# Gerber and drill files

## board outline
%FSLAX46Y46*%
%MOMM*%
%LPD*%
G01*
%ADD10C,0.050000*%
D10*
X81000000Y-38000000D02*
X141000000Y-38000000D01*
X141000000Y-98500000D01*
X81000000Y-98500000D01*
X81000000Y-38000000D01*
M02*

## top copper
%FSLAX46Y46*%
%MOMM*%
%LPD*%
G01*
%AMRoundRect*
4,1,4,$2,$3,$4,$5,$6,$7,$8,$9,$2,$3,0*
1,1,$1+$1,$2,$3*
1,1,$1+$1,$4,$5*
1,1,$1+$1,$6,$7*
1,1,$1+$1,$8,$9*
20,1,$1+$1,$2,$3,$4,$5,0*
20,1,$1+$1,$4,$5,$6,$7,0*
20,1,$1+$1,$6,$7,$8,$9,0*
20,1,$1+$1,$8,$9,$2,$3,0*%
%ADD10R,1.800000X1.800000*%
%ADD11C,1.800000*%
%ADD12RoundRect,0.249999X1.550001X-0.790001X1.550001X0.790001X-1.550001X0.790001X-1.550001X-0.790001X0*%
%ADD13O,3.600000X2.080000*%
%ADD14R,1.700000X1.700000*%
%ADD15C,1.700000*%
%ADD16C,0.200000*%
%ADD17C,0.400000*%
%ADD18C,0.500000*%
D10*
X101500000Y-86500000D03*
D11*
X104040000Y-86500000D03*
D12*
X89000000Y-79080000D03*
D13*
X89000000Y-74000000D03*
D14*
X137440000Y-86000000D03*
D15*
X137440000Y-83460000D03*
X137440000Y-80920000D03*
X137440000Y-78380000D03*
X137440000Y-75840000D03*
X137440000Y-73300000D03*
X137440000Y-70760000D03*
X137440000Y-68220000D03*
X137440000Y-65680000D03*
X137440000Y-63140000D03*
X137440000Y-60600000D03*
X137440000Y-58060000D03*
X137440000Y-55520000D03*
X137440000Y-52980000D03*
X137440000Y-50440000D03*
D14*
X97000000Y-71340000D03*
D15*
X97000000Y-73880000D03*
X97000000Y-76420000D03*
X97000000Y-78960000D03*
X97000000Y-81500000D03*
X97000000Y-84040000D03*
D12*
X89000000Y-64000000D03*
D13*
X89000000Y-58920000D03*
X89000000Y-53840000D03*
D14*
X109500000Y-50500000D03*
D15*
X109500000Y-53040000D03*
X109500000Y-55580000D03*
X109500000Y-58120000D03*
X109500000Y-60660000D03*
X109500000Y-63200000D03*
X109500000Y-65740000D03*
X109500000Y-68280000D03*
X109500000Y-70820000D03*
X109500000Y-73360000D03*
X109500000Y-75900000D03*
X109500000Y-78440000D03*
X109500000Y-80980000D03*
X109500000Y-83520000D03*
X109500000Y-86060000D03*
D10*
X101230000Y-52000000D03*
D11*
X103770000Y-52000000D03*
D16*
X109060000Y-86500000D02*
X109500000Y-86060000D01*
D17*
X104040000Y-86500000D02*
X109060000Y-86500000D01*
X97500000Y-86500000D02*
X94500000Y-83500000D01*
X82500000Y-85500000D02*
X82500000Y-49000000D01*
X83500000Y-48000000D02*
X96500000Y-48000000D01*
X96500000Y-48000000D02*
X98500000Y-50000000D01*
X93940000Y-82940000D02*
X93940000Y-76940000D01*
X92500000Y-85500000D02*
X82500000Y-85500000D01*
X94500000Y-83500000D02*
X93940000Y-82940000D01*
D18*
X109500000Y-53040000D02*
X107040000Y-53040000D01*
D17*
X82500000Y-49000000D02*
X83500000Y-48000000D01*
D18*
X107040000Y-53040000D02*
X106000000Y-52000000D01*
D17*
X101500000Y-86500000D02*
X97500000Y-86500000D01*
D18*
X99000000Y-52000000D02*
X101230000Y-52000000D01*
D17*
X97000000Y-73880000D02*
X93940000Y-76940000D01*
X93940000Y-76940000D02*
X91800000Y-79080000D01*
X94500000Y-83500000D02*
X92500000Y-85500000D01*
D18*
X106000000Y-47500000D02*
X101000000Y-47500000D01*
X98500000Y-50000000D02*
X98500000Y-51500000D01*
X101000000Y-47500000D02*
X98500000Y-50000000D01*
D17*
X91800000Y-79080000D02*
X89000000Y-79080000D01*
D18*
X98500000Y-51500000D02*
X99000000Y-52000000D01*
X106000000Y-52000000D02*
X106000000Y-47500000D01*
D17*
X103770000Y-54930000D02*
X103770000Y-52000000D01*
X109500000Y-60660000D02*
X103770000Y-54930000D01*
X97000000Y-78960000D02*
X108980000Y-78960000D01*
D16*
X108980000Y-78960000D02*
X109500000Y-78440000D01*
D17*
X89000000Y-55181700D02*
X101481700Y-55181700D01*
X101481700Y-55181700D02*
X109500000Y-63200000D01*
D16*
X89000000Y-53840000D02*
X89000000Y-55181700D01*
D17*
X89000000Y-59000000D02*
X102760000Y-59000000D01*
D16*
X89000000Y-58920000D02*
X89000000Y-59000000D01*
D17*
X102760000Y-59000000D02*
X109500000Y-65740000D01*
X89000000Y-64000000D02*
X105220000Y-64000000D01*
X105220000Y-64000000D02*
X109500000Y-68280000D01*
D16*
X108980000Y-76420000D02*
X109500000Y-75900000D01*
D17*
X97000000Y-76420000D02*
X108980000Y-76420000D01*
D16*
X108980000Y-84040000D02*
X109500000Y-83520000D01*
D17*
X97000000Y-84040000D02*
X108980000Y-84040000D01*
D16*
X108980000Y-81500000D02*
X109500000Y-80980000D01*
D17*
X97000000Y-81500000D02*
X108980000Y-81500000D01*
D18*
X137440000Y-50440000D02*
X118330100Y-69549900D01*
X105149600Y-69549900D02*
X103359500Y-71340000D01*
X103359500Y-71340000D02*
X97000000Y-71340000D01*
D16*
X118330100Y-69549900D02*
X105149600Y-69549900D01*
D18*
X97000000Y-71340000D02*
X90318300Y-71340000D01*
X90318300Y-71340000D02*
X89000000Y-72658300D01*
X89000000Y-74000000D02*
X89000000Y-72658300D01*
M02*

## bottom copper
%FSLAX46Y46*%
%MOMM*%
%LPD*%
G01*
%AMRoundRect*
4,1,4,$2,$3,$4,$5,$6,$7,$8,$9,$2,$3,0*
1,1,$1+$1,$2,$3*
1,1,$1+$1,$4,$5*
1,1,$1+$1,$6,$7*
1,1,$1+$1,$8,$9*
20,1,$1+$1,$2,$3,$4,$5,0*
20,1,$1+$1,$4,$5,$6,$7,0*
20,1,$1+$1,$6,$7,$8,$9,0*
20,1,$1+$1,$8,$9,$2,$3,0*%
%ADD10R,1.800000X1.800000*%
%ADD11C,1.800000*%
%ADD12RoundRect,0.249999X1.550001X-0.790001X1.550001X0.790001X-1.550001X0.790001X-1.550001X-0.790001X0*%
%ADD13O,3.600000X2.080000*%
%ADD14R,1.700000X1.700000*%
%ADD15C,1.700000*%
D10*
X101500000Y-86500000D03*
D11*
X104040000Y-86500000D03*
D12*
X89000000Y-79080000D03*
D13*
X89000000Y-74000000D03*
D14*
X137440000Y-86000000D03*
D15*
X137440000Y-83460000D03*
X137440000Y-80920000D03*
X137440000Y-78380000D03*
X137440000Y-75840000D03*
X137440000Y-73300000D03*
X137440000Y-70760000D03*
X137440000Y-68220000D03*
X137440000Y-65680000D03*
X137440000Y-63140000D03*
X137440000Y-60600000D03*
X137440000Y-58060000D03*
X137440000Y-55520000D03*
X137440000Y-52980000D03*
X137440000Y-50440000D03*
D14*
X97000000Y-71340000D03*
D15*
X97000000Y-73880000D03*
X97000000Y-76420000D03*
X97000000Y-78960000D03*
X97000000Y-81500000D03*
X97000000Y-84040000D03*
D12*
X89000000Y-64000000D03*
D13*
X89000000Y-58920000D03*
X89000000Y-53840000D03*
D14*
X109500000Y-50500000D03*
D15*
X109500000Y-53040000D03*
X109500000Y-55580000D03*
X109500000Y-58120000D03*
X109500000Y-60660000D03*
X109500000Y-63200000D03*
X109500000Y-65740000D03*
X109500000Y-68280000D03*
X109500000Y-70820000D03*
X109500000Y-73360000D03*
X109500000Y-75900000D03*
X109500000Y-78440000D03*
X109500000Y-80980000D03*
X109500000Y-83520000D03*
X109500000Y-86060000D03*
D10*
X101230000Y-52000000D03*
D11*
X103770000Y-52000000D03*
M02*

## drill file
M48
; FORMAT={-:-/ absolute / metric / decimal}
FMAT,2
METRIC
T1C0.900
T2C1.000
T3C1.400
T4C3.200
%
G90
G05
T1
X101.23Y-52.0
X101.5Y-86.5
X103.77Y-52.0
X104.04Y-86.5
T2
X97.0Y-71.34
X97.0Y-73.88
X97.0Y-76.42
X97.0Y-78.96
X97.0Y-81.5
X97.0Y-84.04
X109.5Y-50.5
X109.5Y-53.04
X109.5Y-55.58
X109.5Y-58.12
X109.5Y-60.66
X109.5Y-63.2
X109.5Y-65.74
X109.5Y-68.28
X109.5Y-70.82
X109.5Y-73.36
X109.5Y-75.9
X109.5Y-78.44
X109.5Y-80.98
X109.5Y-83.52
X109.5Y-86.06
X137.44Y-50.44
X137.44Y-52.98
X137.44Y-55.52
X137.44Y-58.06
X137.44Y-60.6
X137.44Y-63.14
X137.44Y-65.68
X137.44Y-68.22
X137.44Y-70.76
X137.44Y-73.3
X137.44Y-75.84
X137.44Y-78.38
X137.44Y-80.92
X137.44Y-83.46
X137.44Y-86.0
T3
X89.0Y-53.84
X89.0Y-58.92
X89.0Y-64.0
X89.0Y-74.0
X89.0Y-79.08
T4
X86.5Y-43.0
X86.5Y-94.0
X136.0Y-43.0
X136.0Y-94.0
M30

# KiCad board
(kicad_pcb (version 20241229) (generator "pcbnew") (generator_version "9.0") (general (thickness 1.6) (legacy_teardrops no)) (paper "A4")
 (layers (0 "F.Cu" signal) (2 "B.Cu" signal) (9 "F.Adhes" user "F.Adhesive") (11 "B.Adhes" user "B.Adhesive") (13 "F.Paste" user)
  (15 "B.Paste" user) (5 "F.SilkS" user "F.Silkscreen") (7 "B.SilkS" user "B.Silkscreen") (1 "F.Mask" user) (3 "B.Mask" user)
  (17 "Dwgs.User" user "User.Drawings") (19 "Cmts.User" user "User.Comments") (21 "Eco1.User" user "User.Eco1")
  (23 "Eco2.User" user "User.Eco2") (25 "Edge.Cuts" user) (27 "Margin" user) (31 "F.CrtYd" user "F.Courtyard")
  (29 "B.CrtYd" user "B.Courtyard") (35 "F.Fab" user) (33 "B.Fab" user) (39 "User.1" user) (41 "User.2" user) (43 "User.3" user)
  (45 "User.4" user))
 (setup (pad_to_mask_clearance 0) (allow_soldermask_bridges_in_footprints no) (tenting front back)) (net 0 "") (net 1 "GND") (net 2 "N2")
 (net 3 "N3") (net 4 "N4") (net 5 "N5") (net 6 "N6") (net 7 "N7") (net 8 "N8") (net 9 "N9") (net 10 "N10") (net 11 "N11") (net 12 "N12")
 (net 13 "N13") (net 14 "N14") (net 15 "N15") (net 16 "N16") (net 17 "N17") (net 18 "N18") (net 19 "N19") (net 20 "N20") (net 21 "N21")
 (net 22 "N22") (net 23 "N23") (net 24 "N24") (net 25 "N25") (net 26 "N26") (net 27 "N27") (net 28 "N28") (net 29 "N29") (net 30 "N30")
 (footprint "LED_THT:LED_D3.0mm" (layer "F.Cu") (at 101.5 86.5)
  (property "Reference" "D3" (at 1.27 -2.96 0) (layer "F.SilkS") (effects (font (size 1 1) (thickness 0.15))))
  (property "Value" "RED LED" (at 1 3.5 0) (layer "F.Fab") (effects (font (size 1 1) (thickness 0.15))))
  (pad "1" thru_hole rect (at 0 0) (size 1.8 1.8) (drill 0.9) (layers "*.Cu" "*.Mask") (remove_unused_layers no) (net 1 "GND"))
  (pad "2" thru_hole circle (at 2.54 0) (size 1.8 1.8) (drill 0.9) (layers "*.Cu" "*.Mask") (remove_unused_layers no) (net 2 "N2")))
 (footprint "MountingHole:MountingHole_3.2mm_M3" (layer "F.Cu") (at 86.5 94)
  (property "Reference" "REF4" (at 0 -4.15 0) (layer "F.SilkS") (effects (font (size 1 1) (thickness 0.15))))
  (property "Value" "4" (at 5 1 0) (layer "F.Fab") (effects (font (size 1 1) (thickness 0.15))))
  (pad "" np_thru_hole circle (at 0 0) (size 3.2 3.2) (drill 3.2) (layers "*.Cu" "*.Mask")))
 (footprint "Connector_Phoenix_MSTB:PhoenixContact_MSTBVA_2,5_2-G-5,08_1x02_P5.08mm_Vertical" (layer "F.Cu") (at 89 79.08 90)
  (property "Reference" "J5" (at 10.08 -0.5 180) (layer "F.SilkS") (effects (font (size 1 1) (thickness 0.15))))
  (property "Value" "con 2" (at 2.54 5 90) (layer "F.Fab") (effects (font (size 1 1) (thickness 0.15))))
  (pad "1" thru_hole roundrect (at 0 0 90) (size 2.08 3.6) (drill 1.4) (layers "*.Cu" "*.Mask") (remove_unused_layers no)
   (roundrect_rratio 0.120192) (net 1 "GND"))
  (pad "2" thru_hole oval (at 5.08 0 90) (size 2.08 3.6) (drill 1.4) (layers "*.Cu" "*.Mask") (remove_unused_layers no) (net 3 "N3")))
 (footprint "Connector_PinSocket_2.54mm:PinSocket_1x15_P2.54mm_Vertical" (layer "F.Cu") (at 137.44 86 180)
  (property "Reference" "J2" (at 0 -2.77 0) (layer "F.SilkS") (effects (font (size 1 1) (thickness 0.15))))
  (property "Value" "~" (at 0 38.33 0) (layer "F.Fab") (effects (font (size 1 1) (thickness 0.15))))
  (pad "1" thru_hole rect (at 0 0 180) (size 1.7 1.7) (drill 1) (layers "*.Cu" "*.Mask") (remove_unused_layers no) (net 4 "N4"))
  (pad "2" thru_hole circle (at 0 2.54 180) (size 1.7 1.7) (drill 1) (layers "*.Cu" "*.Mask") (remove_unused_layers no) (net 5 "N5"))
  (pad "3" thru_hole circle (at 0 5.08 180) (size 1.7 1.7) (drill 1) (layers "*.Cu" "*.Mask") (remove_unused_layers no) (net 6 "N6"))
  (pad "4" thru_hole circle (at 0 7.62 180) (size 1.7 1.7) (drill 1) (layers "*.Cu" "*.Mask") (remove_unused_layers no) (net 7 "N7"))
  (pad "5" thru_hole circle (at 0 10.16 180) (size 1.7 1.7) (drill 1) (layers "*.Cu" "*.Mask") (remove_unused_layers no) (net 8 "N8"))
  (pad "6" thru_hole circle (at 0 12.7 180) (size 1.7 1.7) (drill 1) (layers "*.Cu" "*.Mask") (remove_unused_layers no) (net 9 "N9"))
  (pad "7" thru_hole circle (at 0 15.24 180) (size 1.7 1.7) (drill 1) (layers "*.Cu" "*.Mask") (remove_unused_layers no) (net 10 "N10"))
  (pad "8" thru_hole circle (at 0 17.78 180) (size 1.7 1.7) (drill 1) (layers "*.Cu" "*.Mask") (remove_unused_layers no) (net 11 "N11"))
  (pad "9" thru_hole circle (at 0 20.32 180) (size 1.7 1.7) (drill 1) (layers "*.Cu" "*.Mask") (remove_unused_layers no) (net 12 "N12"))
  (pad "10" thru_hole circle (at 0 22.86 180) (size 1.7 1.7) (drill 1) (layers "*.Cu" "*.Mask") (remove_unused_layers no) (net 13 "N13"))
  (pad "11" thru_hole circle (at 0 25.4 180) (size 1.7 1.7) (drill 1) (layers "*.Cu" "*.Mask") (remove_unused_layers no) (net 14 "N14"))
  (pad "12" thru_hole circle (at 0 27.94 180) (size 1.7 1.7) (drill 1) (layers "*.Cu" "*.Mask") (remove_unused_layers no) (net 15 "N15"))
  (pad "13" thru_hole circle (at 0 30.48 180) (size 1.7 1.7) (drill 1) (layers "*.Cu" "*.Mask") (remove_unused_layers no) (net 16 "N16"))
  (pad "14" thru_hole circle (at 0 33.02 180) (size 1.7 1.7) (drill 1) (layers "*.Cu" "*.Mask") (remove_unused_layers no) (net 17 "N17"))
  (pad "15" thru_hole circle (at 0 35.56 180) (size 1.7 1.7) (drill 1) (layers "*.Cu" "*.Mask") (remove_unused_layers no) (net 3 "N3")))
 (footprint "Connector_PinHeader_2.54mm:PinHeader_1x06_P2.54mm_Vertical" (layer "F.Cu") (at 97 71.34)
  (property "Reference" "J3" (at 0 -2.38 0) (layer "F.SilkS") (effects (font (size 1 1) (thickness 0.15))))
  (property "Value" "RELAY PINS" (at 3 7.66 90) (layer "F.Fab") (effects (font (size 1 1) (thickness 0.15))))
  (pad "1" thru_hole rect (at 0 0) (size 1.7 1.7) (drill 1) (layers "*.Cu" "*.Mask") (remove_unused_layers no) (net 3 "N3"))
  (pad "2" thru_hole circle (at 0 2.54) (size 1.7 1.7) (drill 1) (layers "*.Cu" "*.Mask") (remove_unused_layers no) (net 1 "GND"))
  (pad "3" thru_hole circle (at 0 5.08) (size 1.7 1.7) (drill 1) (layers "*.Cu" "*.Mask") (remove_unused_layers no) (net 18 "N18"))
  (pad "4" thru_hole circle (at 0 7.62) (size 1.7 1.7) (drill 1) (layers "*.Cu" "*.Mask") (remove_unused_layers no) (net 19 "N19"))
  (pad "5" thru_hole circle (at 0 10.16) (size 1.7 1.7) (drill 1) (layers "*.Cu" "*.Mask") (remove_unused_layers no) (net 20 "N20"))
  (pad "6" thru_hole circle (at 0 12.7) (size 1.7 1.7) (drill 1) (layers "*.Cu" "*.Mask") (remove_unused_layers no) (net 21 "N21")))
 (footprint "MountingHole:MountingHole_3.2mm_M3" (layer "F.Cu") (at 136 43)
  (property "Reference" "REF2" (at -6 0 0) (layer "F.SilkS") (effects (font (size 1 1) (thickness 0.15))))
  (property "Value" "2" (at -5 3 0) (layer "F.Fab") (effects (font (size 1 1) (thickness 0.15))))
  (pad "" np_thru_hole circle (at 0 0) (size 3.2 3.2) (drill 3.2) (layers "*.Cu" "*.Mask")))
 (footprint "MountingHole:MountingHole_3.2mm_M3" (layer "F.Cu") (at 136 94)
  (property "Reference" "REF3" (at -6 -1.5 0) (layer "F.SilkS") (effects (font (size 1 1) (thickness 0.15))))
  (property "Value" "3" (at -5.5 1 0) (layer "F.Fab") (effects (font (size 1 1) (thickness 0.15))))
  (pad "" np_thru_hole circle (at 0 0) (size 3.2 3.2) (drill 3.2) (layers "*.Cu" "*.Mask")))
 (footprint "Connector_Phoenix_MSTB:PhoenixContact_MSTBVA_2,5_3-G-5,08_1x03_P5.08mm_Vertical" (layer "F.Cu") (at 89 64 90)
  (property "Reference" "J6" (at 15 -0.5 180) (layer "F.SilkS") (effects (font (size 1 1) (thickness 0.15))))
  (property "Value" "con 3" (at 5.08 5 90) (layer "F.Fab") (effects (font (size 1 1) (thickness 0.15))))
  (pad "1" thru_hole roundrect (at 0 0 90) (size 2.08 3.6) (drill 1.4) (layers "*.Cu" "*.Mask") (remove_unused_layers no)
   (roundrect_rratio 0.120192) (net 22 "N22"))
  (pad "2" thru_hole oval (at 5.08 0 90) (size 2.08 3.6) (drill 1.4) (layers "*.Cu" "*.Mask") (remove_unused_layers no) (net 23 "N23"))
  (pad "3" thru_hole oval (at 10.16 0 90) (size 2.08 3.6) (drill 1.4) (layers "*.Cu" "*.Mask") (remove_unused_layers no) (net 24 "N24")))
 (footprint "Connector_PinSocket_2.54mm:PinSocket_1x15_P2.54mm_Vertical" (layer "F.Cu") (at 109.5 50.5)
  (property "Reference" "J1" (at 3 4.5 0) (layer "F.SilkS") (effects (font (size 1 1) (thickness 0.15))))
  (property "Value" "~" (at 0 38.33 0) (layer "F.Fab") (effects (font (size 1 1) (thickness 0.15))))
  (pad "1" thru_hole rect (at 0 0) (size 1.7 1.7) (drill 1) (layers "*.Cu" "*.Mask") (remove_unused_layers no) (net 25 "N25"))
  (pad "2" thru_hole circle (at 0 2.54) (size 1.7 1.7) (drill 1) (layers "*.Cu" "*.Mask") (remove_unused_layers no) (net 1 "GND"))
  (pad "3" thru_hole circle (at 0 5.08) (size 1.7 1.7) (drill 1) (layers "*.Cu" "*.Mask") (remove_unused_layers no) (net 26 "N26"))
  (pad "4" thru_hole circle (at 0 7.62) (size 1.7 1.7) (drill 1) (layers "*.Cu" "*.Mask") (remove_unused_layers no) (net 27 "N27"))
  (pad "5" thru_hole circle (at 0 10.16) (size 1.7 1.7) (drill 1) (layers "*.Cu" "*.Mask") (remove_unused_layers no) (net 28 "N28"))
  (pad "6" thru_hole circle (at 0 12.7) (size 1.7 1.7) (drill 1) (layers "*.Cu" "*.Mask") (remove_unused_layers no) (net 24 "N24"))
  (pad "7" thru_hole circle (at 0 15.24) (size 1.7 1.7) (drill 1) (layers "*.Cu" "*.Mask") (remove_unused_layers no) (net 23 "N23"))
  (pad "8" thru_hole circle (at 0 17.78) (size 1.7 1.7) (drill 1) (layers "*.Cu" "*.Mask") (remove_unused_layers no) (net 22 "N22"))
  (pad "9" thru_hole circle (at 0 20.32) (size 1.7 1.7) (drill 1) (layers "*.Cu" "*.Mask") (remove_unused_layers no) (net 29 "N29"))
  (pad "10" thru_hole circle (at 0 22.86) (size 1.7 1.7) (drill 1) (layers "*.Cu" "*.Mask") (remove_unused_layers no) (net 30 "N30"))
  (pad "11" thru_hole circle (at 0 25.4) (size 1.7 1.7) (drill 1) (layers "*.Cu" "*.Mask") (remove_unused_layers no) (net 18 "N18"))
  (pad "12" thru_hole circle (at 0 27.94) (size 1.7 1.7) (drill 1) (layers "*.Cu" "*.Mask") (remove_unused_layers no) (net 19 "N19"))
  (pad "13" thru_hole circle (at 0 30.48) (size 1.7 1.7) (drill 1) (layers "*.Cu" "*.Mask") (remove_unused_layers no) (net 20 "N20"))
  (pad "14" thru_hole circle (at 0 33.02) (size 1.7 1.7) (drill 1) (layers "*.Cu" "*.Mask") (remove_unused_layers no) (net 21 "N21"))
  (pad "15" thru_hole circle (at 0 35.56) (size 1.7 1.7) (drill 1) (layers "*.Cu" "*.Mask") (remove_unused_layers no) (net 2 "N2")))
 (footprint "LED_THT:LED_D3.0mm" (layer "F.Cu") (at 101.23 52)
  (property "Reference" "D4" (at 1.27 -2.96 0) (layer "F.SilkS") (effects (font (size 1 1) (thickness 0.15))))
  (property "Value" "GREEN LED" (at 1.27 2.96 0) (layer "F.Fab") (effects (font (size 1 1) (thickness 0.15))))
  (pad "1" thru_hole rect (at 0 0) (size 1.8 1.8) (drill 0.9) (layers "*.Cu" "*.Mask") (remove_unused_layers no) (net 1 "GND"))
  (pad "2" thru_hole circle (at 2.54 0) (size 1.8 1.8) (drill 0.9) (layers "*.Cu" "*.Mask") (remove_unused_layers no) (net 28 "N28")))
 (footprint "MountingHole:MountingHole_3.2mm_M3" (layer "F.Cu") (at 86.5 43)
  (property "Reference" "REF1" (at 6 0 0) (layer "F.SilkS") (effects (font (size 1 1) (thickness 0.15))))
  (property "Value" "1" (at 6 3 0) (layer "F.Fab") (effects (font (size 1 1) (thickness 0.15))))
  (pad "" np_thru_hole circle (at 0 0) (size 3.2 3.2) (drill 3.2) (layers "*.Cu" "*.Mask")))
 (gr_rect (start 81 38) (end 141 98.5) (stroke (width 0.05) (type default)) (fill no) (layer "Edge.Cuts"))
 (segment (start 109.06 86.5) (end 109.5 86.06) (width 0.2) (layer "F.Cu") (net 2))
 (segment (start 104.04 86.5) (end 109.06 86.5) (width 0.4) (layer "F.Cu") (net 2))
 (segment (start 97.5 86.5) (end 94.5 83.5) (width 0.4) (layer "F.Cu") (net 1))
 (segment (start 82.5 85.5) (end 82.5 49) (width 0.4) (layer "F.Cu") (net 1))
 (segment (start 83.5 48) (end 96.5 48) (width 0.4) (layer "F.Cu") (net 1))
 (segment (start 96.5 48) (end 98.5 50) (width 0.4) (layer "F.Cu") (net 1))
 (segment (start 93.94 82.94) (end 93.94 76.94) (width 0.4) (layer "F.Cu") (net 1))
 (segment (start 92.5 85.5) (end 82.5 85.5) (width 0.4) (layer "F.Cu") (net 1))
 (segment (start 94.5 83.5) (end 93.94 82.94) (width 0.4) (layer "F.Cu") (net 1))
 (segment (start 109.5 53.04) (end 107.04 53.04) (width 0.5) (layer "F.Cu") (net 1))
 (segment (start 82.5 49) (end 83.5 48) (width 0.4) (layer "F.Cu") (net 1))
 (segment (start 107.04 53.04) (end 106 52) (width 0.5) (layer "F.Cu") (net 1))
 (segment (start 101.5 86.5) (end 97.5 86.5) (width 0.4) (layer "F.Cu") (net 1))
 (segment (start 99 52) (end 101.23 52) (width 0.5) (layer "F.Cu") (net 1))
 (segment (start 97 73.88) (end 93.94 76.94) (width 0.4) (layer "F.Cu") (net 1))
 (segment (start 93.94 76.94) (end 91.8 79.08) (width 0.4) (layer "F.Cu") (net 1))
 (segment (start 94.5 83.5) (end 92.5 85.5) (width 0.4) (layer "F.Cu") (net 1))
 (segment (start 106 47.5) (end 101 47.5) (width 0.5) (layer "F.Cu") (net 1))
 (segment (start 98.5 50) (end 98.5 51.5) (width 0.5) (layer "F.Cu") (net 1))
 (segment (start 101 47.5) (end 98.5 50) (width 0.5) (layer "F.Cu") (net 1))
 (segment (start 91.8 79.08) (end 89 79.08) (width 0.4) (layer "F.Cu") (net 1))
 (segment (start 98.5 51.5) (end 99 52) (width 0.5) (layer "F.Cu") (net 1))
 (segment (start 106 52) (end 106 47.5) (width 0.5) (layer "F.Cu") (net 1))
 (segment (start 103.77 54.93) (end 103.77 52) (width 0.4) (layer "F.Cu") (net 28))
 (segment (start 109.5 60.66) (end 103.77 54.93) (width 0.4) (layer "F.Cu") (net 28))
 (segment (start 97 78.96) (end 108.98 78.96) (width 0.4) (layer "F.Cu") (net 19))
 (segment (start 108.98 78.96) (end 109.5 78.44) (width 0.2) (layer "F.Cu") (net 19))
 (segment (start 89 55.1817) (end 101.4817 55.1817) (width 0.4) (layer "F.Cu") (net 24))
 (segment (start 101.4817 55.1817) (end 109.5 63.2) (width 0.4) (layer "F.Cu") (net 24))
 (segment (start 89 53.84) (end 89 55.1817) (width 0.2) (layer "F.Cu") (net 24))
 (segment (start 89 59) (end 102.76 59) (width 0.4) (layer "F.Cu") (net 23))
 (segment (start 89 58.92) (end 89 59) (width 0.2) (layer "F.Cu") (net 23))
 (segment (start 102.76 59) (end 109.5 65.74) (width 0.4) (layer "F.Cu") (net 23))
 (segment (start 89 64) (end 105.22 64) (width 0.4) (layer "F.Cu") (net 22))
 (segment (start 105.22 64) (end 109.5 68.28) (width 0.4) (layer "F.Cu") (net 22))
 (segment (start 108.98 76.42) (end 109.5 75.9) (width 0.2) (layer "F.Cu") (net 18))
 (segment (start 97 76.42) (end 108.98 76.42) (width 0.4) (layer "F.Cu") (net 18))
 (segment (start 108.98 84.04) (end 109.5 83.52) (width 0.2) (layer "F.Cu") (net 21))
 (segment (start 97 84.04) (end 108.98 84.04) (width 0.4) (layer "F.Cu") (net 21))
 (segment (start 108.98 81.5) (end 109.5 80.98) (width 0.2) (layer "F.Cu") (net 20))
 (segment (start 97 81.5) (end 108.98 81.5) (width 0.4) (layer "F.Cu") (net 20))
 (segment (start 137.44 50.44) (end 118.3301 69.5499) (width 0.5) (layer "F.Cu") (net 3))
 (segment (start 105.1496 69.5499) (end 103.3595 71.34) (width 0.5) (layer "F.Cu") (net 3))
 (segment (start 103.3595 71.34) (end 97 71.34) (width 0.5) (layer "F.Cu") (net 3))
 (segment (start 118.3301 69.5499) (end 105.1496 69.5499) (width 0.2) (layer "F.Cu") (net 3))
 (segment (start 97 71.34) (end 90.3183 71.34) (width 0.5) (layer "F.Cu") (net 3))
 (segment (start 90.3183 71.34) (end 89 72.6583) (width 0.5) (layer "F.Cu") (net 3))
 (segment (start 89 74) (end 89 72.6583) (width 0.5) (layer "F.Cu") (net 3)))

